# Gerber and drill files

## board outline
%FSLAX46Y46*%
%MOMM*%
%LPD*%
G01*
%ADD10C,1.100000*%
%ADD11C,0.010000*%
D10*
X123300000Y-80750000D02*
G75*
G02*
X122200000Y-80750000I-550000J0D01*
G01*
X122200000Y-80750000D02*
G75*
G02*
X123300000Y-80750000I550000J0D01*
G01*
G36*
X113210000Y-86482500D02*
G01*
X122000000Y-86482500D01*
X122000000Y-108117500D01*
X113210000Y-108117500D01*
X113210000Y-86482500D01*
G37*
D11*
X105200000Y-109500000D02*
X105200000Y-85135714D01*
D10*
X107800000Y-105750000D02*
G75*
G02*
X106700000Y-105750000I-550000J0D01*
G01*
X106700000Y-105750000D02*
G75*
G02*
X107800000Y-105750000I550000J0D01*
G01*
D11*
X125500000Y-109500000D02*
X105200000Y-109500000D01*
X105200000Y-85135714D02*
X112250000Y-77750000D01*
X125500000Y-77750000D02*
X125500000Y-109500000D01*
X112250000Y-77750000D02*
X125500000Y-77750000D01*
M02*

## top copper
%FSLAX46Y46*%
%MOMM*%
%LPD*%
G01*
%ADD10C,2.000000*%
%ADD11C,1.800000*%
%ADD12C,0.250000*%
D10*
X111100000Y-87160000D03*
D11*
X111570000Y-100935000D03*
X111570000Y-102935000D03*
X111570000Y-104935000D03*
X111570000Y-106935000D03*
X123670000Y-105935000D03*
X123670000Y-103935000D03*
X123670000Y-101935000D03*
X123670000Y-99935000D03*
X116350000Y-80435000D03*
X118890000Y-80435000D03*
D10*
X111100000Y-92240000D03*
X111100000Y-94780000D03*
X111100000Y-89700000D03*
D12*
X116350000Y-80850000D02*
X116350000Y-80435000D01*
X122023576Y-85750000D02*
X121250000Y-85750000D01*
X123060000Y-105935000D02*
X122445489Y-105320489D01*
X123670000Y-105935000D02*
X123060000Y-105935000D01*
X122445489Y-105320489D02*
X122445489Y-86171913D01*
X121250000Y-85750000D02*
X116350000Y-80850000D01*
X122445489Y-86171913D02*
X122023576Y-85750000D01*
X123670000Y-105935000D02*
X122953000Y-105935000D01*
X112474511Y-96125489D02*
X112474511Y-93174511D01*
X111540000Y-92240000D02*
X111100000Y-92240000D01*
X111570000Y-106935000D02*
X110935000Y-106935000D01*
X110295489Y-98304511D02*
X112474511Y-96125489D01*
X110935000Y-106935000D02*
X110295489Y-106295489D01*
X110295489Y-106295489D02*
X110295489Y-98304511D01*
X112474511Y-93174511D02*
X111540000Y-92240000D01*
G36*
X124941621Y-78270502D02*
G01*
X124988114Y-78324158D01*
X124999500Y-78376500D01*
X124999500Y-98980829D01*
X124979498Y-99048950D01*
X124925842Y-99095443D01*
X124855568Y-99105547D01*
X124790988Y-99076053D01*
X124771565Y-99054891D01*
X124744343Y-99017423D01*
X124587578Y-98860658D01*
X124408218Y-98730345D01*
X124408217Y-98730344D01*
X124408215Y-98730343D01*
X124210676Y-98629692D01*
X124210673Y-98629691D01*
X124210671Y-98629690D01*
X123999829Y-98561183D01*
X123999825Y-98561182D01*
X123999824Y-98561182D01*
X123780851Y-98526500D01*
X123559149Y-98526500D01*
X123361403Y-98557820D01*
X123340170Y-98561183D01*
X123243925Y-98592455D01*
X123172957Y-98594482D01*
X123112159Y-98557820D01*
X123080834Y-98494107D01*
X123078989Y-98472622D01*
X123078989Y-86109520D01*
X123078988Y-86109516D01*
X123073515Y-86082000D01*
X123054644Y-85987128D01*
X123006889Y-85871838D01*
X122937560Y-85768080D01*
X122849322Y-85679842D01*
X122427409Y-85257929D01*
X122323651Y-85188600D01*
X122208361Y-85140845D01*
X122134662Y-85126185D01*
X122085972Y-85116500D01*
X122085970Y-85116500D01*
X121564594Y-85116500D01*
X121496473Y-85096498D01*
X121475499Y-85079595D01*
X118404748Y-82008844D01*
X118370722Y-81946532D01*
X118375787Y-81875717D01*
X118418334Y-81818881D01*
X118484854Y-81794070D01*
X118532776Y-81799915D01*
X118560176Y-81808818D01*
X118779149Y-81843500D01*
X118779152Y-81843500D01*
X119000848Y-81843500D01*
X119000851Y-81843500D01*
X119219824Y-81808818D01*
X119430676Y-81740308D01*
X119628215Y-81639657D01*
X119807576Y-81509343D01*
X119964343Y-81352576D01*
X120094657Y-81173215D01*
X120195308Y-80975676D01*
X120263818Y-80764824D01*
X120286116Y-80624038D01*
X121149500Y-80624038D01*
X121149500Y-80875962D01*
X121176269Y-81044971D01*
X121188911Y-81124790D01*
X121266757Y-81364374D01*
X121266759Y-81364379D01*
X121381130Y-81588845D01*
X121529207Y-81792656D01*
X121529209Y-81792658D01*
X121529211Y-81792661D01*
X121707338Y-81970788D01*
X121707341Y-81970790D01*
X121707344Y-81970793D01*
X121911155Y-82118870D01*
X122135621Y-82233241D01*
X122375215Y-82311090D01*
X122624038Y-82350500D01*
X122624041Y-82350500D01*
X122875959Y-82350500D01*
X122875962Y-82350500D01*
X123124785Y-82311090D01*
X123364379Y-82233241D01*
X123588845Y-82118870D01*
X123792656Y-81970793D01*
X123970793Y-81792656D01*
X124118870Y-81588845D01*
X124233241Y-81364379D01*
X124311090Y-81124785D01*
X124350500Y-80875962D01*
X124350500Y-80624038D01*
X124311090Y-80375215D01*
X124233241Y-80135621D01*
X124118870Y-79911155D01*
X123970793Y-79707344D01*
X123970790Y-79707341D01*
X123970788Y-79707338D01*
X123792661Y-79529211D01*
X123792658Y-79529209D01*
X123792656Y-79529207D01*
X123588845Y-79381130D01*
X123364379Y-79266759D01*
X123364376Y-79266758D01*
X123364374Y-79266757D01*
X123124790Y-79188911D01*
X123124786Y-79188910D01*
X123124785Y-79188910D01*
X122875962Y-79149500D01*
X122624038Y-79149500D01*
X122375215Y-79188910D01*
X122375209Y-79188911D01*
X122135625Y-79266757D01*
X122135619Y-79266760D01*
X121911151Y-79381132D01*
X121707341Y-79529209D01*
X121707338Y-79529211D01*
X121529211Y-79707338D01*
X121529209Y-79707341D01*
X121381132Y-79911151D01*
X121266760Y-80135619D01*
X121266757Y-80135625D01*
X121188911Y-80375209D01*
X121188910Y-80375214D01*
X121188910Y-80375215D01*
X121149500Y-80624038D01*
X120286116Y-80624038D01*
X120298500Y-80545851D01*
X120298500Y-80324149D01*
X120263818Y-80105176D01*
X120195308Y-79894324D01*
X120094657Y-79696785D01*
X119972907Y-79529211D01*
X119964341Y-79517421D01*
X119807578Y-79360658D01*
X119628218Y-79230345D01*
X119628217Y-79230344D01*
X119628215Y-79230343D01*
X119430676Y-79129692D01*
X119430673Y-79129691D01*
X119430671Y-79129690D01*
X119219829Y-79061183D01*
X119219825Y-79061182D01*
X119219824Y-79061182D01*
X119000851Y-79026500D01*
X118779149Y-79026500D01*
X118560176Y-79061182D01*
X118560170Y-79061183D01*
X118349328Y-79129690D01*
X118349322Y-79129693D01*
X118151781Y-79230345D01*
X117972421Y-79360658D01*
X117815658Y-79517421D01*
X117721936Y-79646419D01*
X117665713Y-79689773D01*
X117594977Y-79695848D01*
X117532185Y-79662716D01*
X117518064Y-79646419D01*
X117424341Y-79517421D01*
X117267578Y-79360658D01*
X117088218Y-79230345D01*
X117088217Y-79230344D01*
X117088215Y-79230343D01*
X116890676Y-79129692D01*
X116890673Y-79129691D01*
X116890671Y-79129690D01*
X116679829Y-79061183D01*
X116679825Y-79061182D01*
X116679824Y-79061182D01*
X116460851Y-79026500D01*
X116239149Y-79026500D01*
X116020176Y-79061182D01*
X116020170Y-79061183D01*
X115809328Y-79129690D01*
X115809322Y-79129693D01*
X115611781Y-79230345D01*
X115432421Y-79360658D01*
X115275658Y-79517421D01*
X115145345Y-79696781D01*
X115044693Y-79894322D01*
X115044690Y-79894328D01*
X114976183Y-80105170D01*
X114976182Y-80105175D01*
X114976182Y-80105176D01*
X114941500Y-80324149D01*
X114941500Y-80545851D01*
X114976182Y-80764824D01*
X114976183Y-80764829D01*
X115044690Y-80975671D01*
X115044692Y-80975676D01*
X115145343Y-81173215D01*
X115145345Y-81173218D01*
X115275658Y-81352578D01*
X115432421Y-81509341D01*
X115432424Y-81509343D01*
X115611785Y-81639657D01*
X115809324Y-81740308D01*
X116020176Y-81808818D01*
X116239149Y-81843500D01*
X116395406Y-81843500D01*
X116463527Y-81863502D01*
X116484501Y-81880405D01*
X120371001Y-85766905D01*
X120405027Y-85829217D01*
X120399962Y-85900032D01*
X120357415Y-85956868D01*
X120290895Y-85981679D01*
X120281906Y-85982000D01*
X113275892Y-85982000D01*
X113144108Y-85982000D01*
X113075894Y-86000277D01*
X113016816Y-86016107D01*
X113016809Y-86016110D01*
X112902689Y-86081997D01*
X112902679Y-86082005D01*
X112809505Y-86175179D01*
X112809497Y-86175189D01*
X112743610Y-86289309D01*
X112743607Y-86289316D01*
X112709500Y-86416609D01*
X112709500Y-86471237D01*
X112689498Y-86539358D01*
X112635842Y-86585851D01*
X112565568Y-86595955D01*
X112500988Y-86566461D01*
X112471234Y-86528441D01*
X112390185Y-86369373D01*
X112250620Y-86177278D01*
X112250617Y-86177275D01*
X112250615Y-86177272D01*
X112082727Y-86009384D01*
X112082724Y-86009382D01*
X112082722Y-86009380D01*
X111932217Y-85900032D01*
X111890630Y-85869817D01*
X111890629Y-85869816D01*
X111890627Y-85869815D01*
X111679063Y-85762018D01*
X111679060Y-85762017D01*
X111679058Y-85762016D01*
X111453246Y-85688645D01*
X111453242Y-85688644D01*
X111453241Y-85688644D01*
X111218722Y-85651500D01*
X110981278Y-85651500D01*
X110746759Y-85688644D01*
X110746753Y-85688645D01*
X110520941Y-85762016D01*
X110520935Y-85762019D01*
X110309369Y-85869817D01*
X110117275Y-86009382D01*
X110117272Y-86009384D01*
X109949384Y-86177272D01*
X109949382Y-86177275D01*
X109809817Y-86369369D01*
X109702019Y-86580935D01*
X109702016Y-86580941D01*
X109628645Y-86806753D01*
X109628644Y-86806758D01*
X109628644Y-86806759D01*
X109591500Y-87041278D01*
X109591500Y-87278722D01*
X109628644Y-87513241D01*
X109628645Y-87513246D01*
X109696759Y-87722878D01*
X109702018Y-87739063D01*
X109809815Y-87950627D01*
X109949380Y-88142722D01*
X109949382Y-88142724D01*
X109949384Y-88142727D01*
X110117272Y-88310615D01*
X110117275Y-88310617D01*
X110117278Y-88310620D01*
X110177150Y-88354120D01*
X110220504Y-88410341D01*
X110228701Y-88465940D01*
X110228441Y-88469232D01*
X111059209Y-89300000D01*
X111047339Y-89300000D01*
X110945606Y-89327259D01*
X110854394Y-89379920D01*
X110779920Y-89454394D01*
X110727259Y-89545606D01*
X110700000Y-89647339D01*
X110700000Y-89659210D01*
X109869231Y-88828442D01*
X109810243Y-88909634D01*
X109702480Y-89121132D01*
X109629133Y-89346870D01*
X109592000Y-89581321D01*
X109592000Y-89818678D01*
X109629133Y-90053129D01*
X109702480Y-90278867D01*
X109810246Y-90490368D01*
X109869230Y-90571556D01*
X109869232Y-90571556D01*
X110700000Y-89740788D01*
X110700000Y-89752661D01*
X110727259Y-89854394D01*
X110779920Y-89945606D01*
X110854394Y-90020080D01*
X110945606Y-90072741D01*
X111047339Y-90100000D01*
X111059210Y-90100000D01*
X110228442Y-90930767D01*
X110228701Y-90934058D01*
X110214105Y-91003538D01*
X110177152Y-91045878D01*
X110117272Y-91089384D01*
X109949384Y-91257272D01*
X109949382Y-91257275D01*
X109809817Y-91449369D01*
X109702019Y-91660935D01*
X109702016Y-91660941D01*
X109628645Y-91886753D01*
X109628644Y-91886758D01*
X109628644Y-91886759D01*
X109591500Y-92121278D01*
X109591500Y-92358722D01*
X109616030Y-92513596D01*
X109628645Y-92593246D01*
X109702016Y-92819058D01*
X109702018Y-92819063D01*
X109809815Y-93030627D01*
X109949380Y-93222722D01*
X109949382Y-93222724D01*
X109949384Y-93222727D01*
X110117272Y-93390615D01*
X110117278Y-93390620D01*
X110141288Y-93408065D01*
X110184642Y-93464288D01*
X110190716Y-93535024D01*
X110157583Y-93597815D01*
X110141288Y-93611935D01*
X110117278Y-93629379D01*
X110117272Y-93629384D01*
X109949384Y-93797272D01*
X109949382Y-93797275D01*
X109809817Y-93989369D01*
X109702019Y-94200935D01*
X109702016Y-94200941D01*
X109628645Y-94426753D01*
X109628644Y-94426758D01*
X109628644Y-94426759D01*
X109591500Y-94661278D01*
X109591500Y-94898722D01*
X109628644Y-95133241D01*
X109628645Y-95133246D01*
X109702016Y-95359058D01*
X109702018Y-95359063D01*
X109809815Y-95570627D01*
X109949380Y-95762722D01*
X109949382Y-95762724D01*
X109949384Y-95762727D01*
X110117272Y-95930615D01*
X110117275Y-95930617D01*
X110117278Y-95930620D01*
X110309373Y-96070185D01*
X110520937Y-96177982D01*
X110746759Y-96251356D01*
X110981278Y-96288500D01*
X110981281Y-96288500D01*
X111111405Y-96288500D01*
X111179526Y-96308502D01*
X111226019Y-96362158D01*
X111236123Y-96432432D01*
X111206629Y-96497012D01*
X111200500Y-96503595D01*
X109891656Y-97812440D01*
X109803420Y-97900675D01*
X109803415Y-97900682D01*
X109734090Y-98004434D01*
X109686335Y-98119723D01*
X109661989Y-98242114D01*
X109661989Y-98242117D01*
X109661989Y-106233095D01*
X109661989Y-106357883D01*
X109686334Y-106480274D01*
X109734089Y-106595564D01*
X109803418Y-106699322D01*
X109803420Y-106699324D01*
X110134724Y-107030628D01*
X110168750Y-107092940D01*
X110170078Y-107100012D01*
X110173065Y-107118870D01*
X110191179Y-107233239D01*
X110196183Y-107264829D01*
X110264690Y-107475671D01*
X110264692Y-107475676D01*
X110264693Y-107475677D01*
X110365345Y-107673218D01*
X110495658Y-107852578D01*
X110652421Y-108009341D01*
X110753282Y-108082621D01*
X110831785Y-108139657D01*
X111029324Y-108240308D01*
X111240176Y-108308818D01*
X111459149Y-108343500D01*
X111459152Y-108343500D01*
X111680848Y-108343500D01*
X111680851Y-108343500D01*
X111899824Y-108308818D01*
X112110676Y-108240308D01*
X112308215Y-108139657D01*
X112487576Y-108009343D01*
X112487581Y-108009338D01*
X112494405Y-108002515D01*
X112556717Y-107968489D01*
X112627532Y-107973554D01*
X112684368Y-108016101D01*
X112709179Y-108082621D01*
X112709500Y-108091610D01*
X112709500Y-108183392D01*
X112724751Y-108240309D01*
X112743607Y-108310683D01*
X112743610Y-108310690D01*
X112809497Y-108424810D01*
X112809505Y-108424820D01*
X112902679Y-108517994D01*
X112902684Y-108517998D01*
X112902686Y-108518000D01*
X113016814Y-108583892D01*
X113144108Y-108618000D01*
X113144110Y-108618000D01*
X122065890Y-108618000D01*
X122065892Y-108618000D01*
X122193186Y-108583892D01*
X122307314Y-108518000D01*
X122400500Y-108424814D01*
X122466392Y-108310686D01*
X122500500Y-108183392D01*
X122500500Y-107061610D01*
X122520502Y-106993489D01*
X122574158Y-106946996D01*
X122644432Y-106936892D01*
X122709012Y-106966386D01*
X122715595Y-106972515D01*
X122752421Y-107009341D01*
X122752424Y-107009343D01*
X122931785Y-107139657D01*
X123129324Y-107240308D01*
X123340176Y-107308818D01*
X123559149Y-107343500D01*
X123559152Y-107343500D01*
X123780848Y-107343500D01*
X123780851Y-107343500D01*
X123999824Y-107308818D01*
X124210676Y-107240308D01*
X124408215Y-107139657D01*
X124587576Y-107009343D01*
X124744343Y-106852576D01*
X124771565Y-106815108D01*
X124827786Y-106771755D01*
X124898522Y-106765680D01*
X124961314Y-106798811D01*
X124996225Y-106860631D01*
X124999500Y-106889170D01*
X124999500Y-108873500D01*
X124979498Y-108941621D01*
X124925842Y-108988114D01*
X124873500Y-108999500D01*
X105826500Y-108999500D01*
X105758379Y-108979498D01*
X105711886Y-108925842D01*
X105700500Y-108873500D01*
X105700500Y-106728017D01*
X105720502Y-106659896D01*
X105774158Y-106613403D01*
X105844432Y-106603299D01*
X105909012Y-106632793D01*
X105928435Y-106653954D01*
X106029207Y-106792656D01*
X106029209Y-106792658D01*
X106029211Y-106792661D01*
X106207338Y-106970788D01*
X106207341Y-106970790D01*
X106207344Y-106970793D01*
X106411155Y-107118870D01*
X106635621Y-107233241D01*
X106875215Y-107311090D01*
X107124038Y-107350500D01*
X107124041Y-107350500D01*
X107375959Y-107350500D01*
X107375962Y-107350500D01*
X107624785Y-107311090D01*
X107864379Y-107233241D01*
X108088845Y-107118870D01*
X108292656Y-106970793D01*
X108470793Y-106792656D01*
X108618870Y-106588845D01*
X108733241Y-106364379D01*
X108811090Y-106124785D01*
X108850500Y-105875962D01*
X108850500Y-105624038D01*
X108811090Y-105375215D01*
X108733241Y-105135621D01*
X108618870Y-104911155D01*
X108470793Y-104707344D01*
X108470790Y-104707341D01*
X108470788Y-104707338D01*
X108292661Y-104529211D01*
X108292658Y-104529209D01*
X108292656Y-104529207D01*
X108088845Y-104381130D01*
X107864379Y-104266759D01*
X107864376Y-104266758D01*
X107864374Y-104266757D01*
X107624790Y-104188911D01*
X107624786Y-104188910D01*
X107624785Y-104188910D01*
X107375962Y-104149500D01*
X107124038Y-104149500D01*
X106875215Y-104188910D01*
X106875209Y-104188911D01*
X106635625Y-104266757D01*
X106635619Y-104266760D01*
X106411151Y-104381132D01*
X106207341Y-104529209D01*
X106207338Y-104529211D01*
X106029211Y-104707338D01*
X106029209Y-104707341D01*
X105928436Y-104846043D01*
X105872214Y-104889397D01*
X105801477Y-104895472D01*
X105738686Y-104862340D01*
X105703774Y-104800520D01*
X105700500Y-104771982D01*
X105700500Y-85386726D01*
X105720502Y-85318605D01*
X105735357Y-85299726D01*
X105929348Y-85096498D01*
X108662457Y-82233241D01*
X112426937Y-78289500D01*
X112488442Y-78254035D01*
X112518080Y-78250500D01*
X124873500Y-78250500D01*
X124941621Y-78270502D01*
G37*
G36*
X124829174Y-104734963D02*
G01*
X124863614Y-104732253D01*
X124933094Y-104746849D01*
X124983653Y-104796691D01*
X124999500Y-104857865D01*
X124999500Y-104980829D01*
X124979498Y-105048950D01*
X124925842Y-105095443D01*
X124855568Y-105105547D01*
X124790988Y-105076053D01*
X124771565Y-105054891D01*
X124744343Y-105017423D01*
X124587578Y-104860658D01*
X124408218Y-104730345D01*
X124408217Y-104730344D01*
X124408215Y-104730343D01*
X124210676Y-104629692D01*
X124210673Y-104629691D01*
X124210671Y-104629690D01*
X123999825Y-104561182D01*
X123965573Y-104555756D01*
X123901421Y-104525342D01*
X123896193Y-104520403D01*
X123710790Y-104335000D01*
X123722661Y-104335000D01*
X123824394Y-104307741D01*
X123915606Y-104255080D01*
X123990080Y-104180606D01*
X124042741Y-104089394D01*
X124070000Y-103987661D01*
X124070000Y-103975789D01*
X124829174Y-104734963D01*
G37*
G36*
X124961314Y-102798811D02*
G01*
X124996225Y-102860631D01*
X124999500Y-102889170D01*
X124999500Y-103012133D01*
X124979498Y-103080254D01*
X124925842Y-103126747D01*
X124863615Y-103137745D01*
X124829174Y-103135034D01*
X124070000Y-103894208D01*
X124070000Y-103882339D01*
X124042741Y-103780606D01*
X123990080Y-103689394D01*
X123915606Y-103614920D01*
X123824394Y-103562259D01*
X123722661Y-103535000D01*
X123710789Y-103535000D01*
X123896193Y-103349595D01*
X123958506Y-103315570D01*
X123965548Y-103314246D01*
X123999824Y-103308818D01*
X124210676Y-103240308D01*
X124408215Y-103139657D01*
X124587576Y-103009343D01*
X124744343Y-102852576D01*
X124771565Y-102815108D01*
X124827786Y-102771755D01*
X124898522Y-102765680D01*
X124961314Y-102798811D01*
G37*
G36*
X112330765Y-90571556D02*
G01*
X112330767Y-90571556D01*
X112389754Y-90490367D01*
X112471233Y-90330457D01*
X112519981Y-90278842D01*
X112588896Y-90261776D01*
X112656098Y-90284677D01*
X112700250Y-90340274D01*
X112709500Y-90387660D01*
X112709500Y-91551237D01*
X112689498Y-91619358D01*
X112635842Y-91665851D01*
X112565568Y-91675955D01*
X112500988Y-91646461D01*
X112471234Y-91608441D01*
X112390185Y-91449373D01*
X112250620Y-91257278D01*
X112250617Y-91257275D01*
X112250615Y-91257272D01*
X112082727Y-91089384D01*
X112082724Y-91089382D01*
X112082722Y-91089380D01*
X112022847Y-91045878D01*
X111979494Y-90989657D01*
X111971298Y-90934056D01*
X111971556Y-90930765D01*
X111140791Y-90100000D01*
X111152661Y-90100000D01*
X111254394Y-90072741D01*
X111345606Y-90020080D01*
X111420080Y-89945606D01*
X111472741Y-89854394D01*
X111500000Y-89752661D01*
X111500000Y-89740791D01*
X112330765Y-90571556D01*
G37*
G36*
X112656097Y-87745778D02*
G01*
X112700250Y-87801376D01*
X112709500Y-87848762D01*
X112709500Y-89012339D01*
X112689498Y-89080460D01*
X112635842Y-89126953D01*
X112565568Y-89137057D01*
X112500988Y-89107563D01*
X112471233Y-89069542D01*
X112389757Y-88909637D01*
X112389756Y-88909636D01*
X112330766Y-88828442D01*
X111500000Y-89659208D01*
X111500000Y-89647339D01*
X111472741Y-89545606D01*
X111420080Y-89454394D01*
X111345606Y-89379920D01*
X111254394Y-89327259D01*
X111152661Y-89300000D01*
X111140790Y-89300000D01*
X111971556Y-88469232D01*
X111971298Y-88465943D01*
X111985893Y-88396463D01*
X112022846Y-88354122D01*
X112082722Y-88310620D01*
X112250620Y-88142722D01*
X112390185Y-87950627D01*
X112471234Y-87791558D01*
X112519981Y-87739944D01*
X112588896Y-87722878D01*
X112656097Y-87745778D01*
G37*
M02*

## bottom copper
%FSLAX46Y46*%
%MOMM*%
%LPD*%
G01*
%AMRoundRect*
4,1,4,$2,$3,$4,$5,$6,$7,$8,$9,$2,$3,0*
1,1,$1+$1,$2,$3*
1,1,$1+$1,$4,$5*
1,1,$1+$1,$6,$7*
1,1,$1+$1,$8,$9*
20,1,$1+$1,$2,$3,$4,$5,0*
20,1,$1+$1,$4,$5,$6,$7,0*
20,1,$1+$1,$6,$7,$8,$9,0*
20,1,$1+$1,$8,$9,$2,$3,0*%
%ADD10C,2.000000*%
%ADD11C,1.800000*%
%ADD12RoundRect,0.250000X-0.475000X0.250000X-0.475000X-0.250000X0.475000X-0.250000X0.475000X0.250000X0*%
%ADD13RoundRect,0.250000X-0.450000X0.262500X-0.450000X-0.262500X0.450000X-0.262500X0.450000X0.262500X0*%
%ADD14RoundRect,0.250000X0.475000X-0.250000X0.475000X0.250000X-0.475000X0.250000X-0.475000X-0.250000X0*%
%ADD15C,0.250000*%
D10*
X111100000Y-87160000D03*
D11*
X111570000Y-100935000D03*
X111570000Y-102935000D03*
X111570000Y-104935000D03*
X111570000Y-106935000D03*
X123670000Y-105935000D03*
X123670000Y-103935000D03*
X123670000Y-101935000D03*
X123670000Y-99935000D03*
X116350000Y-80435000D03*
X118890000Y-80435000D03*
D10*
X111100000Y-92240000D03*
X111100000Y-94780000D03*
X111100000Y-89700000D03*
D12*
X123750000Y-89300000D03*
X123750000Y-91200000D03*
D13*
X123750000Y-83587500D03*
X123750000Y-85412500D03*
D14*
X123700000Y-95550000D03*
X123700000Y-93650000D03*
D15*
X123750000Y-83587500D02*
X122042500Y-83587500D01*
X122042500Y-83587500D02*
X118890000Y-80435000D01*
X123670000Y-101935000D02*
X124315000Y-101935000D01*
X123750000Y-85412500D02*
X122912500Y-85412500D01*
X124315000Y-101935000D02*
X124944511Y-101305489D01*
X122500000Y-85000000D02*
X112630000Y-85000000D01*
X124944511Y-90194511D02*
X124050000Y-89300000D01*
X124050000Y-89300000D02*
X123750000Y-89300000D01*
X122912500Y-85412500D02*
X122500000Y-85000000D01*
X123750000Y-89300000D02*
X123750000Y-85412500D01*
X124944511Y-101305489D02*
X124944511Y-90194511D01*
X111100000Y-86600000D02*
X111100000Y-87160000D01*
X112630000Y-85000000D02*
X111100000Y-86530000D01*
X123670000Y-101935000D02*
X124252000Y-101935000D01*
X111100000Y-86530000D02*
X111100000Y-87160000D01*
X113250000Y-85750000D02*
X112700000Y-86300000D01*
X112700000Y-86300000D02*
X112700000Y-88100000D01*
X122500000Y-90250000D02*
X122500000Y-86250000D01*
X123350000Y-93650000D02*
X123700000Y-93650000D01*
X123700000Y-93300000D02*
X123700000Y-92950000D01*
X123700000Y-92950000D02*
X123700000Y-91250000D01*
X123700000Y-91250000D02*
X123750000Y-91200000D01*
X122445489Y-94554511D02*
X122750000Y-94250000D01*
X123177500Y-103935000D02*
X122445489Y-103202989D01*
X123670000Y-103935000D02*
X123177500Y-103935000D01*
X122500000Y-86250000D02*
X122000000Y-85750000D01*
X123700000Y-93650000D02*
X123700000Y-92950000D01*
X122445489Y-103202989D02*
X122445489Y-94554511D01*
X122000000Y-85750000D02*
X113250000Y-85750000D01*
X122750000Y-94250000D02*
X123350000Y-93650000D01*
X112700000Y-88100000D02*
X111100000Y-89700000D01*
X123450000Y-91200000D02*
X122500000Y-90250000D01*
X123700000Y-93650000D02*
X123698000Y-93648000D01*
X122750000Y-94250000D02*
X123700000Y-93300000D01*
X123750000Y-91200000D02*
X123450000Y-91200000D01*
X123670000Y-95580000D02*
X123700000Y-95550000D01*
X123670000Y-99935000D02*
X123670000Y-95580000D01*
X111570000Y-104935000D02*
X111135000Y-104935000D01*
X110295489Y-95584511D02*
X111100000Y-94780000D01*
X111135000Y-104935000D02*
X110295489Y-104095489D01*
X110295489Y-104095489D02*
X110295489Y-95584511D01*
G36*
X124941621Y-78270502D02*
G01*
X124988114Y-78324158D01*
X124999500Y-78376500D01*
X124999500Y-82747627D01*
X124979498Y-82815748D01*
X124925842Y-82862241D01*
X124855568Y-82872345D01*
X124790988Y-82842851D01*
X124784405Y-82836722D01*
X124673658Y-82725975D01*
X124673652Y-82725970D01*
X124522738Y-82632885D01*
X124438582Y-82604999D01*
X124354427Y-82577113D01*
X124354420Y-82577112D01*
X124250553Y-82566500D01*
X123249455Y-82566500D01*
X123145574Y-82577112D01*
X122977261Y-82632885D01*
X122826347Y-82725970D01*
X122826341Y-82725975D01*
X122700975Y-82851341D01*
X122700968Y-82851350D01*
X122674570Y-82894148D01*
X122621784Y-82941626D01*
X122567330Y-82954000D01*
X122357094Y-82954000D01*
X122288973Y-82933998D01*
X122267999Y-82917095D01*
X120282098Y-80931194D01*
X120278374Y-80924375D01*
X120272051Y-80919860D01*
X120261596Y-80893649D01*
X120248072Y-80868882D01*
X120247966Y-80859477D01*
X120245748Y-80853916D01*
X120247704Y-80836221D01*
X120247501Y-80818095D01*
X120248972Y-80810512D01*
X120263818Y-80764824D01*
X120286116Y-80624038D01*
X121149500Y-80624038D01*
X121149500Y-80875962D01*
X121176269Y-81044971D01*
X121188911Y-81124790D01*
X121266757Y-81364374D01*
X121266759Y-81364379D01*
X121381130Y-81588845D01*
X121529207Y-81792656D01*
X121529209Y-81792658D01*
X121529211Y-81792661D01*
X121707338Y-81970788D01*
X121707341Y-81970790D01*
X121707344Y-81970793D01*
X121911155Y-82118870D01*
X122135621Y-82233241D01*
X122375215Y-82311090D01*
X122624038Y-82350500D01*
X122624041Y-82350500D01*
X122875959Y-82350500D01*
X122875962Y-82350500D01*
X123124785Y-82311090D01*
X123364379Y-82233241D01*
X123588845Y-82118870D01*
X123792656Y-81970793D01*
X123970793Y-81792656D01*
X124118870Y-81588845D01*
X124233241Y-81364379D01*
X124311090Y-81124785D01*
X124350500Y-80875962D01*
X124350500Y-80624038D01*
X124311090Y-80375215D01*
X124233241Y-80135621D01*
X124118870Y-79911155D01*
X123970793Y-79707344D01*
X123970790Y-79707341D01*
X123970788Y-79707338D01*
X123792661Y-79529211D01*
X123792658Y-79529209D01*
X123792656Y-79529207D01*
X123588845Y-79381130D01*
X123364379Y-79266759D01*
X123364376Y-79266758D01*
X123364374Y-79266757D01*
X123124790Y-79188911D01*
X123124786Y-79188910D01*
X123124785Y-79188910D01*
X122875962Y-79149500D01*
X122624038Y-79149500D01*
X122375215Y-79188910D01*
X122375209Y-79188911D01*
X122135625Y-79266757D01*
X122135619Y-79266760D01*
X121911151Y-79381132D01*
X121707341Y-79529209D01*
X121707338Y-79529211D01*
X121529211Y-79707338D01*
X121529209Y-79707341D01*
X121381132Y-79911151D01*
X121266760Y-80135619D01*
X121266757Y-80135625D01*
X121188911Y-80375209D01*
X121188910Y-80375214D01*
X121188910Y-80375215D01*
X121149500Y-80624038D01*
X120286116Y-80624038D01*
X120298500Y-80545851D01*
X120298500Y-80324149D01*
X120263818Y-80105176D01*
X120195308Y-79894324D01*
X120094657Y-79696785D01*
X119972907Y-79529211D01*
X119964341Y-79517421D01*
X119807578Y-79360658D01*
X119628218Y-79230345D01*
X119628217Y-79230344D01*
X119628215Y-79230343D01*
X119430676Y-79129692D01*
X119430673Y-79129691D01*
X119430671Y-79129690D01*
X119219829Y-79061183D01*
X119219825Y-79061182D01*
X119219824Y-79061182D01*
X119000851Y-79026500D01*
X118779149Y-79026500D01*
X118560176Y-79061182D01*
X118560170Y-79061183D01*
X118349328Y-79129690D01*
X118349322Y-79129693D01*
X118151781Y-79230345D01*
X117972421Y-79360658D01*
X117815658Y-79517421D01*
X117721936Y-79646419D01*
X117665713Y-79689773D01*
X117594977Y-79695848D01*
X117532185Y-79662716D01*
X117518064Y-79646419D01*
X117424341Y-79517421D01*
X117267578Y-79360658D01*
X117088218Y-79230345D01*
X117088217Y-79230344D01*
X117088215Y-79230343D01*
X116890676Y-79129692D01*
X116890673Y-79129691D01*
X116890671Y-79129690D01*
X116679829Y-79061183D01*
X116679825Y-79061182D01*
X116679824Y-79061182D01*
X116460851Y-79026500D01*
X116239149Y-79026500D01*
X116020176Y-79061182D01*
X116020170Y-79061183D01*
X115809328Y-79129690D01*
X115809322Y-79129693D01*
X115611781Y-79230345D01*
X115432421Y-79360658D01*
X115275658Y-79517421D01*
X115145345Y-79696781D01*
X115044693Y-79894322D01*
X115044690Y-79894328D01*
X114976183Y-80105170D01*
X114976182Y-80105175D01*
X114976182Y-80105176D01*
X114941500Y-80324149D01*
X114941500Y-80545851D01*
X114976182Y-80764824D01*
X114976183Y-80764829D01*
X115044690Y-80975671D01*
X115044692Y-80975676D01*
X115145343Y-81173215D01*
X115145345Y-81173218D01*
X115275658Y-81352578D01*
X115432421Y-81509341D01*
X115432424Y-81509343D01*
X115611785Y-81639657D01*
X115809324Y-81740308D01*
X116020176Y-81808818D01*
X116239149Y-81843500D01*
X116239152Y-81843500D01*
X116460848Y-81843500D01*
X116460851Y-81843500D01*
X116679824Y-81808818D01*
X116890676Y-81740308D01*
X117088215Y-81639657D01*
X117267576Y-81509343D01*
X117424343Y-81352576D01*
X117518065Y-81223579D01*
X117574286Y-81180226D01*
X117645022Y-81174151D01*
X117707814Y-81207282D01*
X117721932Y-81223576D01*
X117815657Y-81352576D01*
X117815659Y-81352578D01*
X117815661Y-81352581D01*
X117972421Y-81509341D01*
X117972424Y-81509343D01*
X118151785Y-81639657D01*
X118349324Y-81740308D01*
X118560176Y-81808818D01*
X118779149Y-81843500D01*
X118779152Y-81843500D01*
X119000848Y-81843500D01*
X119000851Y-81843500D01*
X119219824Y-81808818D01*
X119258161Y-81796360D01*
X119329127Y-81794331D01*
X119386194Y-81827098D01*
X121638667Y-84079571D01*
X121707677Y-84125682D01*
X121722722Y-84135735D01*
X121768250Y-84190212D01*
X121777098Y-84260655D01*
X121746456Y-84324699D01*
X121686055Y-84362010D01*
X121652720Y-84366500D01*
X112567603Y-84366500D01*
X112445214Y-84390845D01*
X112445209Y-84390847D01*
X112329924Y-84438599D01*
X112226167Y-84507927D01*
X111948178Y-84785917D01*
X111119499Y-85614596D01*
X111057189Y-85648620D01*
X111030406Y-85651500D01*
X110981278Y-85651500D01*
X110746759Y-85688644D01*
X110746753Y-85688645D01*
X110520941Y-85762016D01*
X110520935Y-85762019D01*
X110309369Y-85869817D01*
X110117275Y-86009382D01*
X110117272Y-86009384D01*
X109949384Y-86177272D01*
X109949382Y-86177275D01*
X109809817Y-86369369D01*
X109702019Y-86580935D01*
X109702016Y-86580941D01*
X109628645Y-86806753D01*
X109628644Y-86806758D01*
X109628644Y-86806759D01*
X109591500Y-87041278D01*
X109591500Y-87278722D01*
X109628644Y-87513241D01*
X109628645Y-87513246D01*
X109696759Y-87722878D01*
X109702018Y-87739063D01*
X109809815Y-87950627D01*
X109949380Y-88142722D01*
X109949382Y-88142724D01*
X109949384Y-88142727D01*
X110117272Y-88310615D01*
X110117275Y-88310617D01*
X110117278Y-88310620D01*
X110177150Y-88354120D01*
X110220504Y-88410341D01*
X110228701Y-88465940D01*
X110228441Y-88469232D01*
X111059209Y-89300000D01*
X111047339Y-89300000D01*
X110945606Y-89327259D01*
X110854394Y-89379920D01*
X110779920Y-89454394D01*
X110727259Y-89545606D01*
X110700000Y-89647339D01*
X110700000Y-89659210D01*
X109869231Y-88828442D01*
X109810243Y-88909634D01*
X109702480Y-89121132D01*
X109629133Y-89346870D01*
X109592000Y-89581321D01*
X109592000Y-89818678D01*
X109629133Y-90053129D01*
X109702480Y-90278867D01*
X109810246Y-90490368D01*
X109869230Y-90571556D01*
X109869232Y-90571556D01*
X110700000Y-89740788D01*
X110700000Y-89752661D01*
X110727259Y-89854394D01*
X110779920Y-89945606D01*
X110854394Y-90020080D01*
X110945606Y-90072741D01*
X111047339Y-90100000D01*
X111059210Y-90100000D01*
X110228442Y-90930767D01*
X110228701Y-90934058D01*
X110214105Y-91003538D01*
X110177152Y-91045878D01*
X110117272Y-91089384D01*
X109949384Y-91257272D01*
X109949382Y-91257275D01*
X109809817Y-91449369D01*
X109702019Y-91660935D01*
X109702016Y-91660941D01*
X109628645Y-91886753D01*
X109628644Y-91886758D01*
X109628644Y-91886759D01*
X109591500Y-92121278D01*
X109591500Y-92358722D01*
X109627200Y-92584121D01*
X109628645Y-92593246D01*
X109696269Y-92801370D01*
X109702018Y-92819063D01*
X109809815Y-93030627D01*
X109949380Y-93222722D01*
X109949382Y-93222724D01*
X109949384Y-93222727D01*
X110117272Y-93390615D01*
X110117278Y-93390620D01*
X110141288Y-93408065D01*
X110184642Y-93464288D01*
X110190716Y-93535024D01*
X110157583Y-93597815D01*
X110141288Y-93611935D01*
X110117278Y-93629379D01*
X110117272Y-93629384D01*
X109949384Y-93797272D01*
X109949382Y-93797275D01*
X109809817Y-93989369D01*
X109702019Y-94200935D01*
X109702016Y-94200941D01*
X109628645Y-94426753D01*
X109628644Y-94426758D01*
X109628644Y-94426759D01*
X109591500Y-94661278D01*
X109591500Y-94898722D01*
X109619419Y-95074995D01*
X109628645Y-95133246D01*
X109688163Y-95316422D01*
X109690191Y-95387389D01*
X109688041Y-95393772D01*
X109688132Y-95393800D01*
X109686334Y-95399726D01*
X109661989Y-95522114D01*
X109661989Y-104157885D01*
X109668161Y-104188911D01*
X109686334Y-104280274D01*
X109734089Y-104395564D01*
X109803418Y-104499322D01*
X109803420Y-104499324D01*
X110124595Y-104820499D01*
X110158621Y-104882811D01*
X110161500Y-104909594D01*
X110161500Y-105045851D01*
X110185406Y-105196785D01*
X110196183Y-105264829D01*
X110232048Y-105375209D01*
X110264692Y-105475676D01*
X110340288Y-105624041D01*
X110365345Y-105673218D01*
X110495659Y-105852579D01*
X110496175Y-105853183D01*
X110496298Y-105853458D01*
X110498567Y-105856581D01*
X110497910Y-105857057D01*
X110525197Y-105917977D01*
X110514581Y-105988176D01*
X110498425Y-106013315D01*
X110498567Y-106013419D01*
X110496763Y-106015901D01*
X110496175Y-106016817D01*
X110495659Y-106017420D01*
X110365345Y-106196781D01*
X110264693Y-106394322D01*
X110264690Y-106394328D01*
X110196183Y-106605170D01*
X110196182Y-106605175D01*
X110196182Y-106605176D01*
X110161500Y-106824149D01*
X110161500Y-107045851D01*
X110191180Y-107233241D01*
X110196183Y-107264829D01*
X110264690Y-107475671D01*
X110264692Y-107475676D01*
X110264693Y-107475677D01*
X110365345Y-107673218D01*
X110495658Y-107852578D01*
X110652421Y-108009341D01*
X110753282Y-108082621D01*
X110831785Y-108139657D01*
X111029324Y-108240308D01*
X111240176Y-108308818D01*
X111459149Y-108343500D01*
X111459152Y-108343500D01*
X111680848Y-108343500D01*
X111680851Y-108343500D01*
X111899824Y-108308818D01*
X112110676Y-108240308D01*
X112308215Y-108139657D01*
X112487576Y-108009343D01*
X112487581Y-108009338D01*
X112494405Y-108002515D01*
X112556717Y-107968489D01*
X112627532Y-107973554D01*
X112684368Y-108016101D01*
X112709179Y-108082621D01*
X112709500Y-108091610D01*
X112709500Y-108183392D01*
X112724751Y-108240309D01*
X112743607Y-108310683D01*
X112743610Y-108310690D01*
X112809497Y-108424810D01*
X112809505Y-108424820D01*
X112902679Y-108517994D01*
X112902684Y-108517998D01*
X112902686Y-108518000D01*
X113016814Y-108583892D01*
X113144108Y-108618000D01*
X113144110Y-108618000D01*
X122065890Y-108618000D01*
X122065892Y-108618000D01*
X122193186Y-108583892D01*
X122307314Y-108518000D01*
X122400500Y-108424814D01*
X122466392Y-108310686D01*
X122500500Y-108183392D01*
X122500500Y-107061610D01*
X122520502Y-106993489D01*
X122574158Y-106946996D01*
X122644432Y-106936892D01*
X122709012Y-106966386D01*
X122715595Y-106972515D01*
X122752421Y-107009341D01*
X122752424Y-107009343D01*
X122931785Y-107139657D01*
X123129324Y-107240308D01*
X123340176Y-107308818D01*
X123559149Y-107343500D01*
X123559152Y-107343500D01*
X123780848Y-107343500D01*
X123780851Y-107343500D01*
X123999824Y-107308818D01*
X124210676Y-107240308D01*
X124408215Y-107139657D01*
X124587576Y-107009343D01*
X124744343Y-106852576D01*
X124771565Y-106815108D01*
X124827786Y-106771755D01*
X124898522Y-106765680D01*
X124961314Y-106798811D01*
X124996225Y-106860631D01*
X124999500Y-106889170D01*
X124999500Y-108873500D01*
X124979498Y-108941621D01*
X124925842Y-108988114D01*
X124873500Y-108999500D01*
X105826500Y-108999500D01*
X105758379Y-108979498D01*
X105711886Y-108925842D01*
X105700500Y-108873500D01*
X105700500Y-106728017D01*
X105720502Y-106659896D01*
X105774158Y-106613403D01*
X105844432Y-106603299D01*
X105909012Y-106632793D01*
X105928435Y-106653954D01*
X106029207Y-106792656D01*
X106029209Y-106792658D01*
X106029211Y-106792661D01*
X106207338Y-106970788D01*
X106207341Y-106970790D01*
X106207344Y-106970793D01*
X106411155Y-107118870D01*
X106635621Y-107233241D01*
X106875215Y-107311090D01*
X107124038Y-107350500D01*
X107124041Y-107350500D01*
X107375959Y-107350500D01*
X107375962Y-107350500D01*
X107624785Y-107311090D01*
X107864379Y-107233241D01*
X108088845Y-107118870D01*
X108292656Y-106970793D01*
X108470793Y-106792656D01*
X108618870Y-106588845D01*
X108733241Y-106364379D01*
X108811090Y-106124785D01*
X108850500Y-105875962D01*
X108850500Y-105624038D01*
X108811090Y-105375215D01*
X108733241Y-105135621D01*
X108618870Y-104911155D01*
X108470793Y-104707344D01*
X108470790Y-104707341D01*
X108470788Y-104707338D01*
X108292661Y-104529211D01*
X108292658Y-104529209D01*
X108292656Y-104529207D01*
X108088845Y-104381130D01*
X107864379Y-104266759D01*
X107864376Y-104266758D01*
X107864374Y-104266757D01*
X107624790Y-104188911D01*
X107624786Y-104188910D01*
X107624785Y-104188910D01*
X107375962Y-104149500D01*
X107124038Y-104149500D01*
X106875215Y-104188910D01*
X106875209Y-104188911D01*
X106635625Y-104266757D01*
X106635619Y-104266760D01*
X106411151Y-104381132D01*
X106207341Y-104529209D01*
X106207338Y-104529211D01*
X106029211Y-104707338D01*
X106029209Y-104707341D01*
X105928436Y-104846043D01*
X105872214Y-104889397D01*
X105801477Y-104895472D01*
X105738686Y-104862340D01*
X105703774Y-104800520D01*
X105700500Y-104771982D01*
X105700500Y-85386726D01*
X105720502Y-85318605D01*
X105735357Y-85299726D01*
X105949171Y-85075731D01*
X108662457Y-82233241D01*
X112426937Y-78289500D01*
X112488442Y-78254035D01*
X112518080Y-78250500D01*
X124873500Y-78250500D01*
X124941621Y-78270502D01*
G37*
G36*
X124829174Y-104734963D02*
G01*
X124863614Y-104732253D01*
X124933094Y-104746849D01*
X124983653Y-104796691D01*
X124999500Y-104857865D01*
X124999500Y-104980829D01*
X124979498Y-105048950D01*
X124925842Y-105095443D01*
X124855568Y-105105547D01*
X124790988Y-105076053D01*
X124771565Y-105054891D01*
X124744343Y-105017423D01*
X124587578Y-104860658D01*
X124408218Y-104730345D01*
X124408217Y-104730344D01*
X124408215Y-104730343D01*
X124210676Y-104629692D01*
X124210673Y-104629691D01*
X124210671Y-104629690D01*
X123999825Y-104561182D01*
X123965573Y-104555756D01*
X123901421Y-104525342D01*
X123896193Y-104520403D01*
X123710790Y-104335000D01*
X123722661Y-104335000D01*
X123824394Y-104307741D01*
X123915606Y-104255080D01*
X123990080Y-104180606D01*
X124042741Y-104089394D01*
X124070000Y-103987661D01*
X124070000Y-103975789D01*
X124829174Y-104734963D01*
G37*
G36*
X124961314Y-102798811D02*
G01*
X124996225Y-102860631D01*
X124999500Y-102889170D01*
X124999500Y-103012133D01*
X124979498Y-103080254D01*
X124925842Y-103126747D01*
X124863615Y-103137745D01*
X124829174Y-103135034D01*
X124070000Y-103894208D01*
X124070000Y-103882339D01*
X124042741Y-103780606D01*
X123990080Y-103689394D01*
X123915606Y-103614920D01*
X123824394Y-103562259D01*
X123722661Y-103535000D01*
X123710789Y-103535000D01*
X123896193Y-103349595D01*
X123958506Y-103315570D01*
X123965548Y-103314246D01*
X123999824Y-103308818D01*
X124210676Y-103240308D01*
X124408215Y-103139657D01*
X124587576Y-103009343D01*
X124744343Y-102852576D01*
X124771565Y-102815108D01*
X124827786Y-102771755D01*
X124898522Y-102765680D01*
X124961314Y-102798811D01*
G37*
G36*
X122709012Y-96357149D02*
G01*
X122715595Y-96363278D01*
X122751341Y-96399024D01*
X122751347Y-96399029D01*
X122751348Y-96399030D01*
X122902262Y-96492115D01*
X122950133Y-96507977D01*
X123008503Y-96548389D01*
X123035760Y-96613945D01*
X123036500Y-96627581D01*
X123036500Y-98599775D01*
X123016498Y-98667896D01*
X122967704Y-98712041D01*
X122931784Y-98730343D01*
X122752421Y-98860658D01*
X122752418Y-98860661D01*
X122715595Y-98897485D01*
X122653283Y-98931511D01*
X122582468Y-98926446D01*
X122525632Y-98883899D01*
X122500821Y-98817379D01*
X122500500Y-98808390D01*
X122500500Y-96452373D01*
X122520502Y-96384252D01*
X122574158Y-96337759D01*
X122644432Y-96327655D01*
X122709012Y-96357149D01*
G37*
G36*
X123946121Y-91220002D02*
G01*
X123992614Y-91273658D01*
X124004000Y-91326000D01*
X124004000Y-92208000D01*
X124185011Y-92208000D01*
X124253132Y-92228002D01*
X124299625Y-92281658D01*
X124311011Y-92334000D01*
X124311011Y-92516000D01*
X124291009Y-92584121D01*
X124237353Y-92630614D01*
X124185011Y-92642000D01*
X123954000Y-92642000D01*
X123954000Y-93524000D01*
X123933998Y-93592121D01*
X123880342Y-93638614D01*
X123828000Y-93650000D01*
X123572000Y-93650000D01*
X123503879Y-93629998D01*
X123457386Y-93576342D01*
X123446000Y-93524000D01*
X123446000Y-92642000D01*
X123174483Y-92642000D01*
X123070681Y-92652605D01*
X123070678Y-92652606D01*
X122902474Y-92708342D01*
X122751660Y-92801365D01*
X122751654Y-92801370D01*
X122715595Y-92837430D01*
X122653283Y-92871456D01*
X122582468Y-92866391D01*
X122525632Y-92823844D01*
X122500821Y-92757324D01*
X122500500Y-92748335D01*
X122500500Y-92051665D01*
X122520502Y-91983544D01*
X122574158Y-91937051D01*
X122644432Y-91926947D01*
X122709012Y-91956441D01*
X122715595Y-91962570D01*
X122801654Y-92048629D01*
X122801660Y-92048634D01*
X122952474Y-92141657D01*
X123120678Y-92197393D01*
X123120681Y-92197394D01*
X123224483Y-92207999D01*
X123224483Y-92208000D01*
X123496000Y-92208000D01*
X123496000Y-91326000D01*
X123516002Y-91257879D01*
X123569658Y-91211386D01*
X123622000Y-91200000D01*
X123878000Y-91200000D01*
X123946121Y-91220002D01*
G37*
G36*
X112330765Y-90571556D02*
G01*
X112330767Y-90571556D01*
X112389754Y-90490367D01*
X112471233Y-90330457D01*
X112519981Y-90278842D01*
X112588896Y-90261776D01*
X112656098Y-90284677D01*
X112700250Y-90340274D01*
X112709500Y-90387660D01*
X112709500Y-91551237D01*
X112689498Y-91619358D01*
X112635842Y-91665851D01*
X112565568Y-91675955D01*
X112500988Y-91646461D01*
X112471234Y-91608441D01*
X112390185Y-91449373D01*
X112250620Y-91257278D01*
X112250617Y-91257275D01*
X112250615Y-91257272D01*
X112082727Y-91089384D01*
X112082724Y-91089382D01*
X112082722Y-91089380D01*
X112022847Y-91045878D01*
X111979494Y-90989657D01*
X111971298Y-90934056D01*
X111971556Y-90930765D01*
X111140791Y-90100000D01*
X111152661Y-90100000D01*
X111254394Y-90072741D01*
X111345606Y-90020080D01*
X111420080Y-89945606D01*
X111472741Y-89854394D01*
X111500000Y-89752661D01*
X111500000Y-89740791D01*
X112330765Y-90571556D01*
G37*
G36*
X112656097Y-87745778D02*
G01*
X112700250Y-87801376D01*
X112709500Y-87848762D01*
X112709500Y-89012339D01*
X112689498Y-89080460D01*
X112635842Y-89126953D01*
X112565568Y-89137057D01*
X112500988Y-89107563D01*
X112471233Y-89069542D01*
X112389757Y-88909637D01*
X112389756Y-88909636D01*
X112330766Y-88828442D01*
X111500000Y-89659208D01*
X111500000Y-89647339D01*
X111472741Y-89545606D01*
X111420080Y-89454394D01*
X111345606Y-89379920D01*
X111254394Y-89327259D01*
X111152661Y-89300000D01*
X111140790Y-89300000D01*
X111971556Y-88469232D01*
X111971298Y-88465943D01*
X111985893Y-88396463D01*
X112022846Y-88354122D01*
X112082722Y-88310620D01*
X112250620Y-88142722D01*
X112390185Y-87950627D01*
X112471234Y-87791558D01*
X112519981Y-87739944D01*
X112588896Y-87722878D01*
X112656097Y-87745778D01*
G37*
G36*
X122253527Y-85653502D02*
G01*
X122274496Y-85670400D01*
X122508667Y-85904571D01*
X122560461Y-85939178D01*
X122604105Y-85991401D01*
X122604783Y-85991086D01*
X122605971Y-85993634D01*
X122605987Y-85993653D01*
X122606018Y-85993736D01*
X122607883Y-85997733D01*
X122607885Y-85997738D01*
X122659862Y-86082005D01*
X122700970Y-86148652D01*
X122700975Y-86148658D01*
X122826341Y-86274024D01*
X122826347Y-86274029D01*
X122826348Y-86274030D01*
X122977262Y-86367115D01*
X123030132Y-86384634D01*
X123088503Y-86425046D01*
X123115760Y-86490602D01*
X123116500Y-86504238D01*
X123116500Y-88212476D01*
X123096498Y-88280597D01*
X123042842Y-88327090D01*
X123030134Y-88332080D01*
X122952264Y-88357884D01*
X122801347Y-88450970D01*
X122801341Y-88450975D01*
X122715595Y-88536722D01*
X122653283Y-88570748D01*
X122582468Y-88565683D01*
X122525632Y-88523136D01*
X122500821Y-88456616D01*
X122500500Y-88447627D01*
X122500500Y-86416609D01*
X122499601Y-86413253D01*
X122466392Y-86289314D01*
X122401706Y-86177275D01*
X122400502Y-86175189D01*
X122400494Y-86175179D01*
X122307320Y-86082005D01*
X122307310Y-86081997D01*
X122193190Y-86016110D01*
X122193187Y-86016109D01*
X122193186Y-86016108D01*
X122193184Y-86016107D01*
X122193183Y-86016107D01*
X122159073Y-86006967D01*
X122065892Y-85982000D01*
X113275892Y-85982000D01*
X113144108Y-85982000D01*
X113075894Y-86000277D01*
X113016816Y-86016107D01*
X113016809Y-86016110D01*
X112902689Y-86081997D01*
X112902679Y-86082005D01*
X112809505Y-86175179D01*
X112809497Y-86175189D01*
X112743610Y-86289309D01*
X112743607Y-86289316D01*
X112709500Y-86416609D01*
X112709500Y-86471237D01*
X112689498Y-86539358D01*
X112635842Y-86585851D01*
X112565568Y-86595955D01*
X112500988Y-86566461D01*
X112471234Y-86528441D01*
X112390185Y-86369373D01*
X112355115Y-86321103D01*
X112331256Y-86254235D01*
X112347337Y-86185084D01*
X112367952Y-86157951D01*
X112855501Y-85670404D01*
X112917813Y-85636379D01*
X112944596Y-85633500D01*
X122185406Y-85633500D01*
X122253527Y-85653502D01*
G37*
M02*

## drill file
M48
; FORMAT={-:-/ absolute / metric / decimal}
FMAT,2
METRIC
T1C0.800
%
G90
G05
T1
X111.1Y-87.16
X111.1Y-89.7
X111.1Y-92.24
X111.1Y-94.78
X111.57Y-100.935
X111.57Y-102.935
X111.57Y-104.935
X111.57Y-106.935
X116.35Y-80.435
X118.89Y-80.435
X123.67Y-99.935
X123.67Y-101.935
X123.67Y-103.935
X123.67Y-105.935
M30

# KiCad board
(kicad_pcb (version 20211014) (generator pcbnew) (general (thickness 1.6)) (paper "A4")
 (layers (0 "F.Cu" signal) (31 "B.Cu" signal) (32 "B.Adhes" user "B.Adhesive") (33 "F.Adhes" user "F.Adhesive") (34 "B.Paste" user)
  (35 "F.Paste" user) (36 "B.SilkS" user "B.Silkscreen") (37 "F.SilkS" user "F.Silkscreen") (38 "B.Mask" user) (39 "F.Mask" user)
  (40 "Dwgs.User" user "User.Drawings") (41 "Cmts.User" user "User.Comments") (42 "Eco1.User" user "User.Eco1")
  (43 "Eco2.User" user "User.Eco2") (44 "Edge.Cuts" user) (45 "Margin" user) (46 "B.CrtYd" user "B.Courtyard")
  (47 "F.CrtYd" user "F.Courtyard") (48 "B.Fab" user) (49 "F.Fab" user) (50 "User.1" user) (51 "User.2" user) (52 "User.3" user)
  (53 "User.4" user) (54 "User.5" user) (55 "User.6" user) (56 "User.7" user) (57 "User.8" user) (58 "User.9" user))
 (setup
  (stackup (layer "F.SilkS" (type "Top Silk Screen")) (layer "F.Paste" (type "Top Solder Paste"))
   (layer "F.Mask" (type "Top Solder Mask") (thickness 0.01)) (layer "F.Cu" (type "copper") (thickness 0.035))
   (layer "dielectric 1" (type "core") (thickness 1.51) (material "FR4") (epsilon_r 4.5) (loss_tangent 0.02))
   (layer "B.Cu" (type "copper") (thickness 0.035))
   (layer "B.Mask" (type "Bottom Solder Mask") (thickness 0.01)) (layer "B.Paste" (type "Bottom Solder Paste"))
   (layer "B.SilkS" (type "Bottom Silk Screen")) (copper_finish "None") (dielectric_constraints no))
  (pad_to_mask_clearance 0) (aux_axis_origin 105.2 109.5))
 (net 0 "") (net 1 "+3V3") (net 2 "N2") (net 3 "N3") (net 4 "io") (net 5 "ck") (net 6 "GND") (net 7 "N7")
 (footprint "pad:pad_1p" (layer "F.Cu") (at 111.1 87.16)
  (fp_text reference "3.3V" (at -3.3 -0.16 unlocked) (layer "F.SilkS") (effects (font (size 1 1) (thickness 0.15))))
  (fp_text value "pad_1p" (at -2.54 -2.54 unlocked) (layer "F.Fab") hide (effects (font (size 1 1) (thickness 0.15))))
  (pad "1" thru_hole circle (at 0 0) (size 2 2) (drill 0.8) (layers *.Cu *.Mask) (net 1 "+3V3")))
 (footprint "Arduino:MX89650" (layer "F.Cu") (at 117.62 102.935)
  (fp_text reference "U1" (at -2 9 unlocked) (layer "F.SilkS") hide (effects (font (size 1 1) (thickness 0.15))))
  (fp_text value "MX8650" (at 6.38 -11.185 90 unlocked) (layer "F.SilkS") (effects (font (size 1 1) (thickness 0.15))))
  (pad "1" thru_hole circle (at -6.05 -2) (size 1.8 1.8) (drill 0.8) (layers *.Cu *.Mask) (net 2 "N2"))
  (pad "2" thru_hole circle (at -6.05 0) (size 1.8 1.8) (drill 0.8) (layers *.Cu *.Mask) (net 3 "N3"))
  (pad "3" thru_hole circle (at -6.05 2) (size 1.8 1.8) (drill 0.8) (layers *.Cu *.Mask) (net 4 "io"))
  (pad "4" thru_hole circle (at -6.05 4) (size 1.8 1.8) (drill 0.8) (layers *.Cu *.Mask) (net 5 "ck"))
  (pad "5" thru_hole circle (at 6.05 3) (size 1.8 1.8) (drill 0.8) (layers *.Cu *.Mask))
  (pad "6" thru_hole circle (at 6.05 1) (size 1.8 1.8) (drill 0.8) (layers *.Cu *.Mask) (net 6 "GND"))
  (pad "7" thru_hole circle (at 6.05 -1) (size 1.8 1.8) (drill 0.8) (layers *.Cu *.Mask) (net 1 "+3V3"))
  (pad "8" thru_hole circle (at 6.05 -3) (size 1.8 1.8) (drill 0.8) (layers *.Cu *.Mask) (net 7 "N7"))
  (pad "9" thru_hole circle (at -1.27 -22.5) (size 1.8 1.8) (drill 0.8) (layers *.Cu *.Mask))
  (pad "10" thru_hole circle (at 1.27 -22.5) (size 1.8 1.8) (drill 0.8) (layers *.Cu *.Mask)))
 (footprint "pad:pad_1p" (layer "F.Cu") (at 111.1 92.24)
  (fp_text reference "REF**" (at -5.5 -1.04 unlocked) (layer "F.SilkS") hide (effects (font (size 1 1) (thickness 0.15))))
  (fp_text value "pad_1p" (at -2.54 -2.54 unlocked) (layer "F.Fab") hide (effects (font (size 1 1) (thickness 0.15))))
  (pad "1" thru_hole circle (at 0 0) (size 2 2) (drill 0.8) (layers *.Cu *.Mask) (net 5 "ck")))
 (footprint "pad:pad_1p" (layer "F.Cu") (at 111.1 94.78)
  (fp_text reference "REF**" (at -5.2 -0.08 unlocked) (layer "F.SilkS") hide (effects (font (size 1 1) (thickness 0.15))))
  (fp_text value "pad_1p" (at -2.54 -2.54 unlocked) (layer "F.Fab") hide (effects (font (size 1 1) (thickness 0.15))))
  (pad "1" thru_hole circle (at 0 0) (size 2 2) (drill 0.8) (layers *.Cu *.Mask) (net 4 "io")))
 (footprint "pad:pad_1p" (layer "F.Cu") (at 111.1 89.7)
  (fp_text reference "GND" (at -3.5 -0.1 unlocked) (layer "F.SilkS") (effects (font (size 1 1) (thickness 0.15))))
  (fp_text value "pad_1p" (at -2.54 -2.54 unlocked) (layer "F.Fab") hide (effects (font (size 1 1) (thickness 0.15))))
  (pad "1" thru_hole circle (at 0 0) (size 2 2) (drill 0.8) (layers *.Cu *.Mask) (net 6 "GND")))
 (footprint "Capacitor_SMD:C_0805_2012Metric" (layer "B.Cu") (at 123.75 90.25 -90)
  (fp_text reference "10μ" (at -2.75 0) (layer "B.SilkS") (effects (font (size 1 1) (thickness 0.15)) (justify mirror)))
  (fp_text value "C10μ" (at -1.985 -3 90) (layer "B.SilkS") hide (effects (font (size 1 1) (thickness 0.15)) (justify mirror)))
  (pad "1" smd roundrect (at -0.95 0 270) (size 1 1.45) (layers "B.Cu" "B.Paste" "B.Mask") (roundrect_rratio 0.25) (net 1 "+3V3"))
  (pad "2" smd roundrect (at 0.95 0 270) (size 1 1.45) (layers "B.Cu" "B.Paste" "B.Mask") (roundrect_rratio 0.25) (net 6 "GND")))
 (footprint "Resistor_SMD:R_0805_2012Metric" (layer "B.Cu") (at 123.75 84.5 -90)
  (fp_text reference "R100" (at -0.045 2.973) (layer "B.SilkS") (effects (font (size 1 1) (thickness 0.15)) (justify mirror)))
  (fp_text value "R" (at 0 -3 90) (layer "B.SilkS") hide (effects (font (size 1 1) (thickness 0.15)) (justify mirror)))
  (pad "1" smd roundrect (at -0.9125 0 270) (size 1.025 1.4) (layers "B.Cu" "B.Paste" "B.Mask") (roundrect_rratio 0.243902439))
  (pad "2" smd roundrect (at 0.9125 0 270) (size 1.025 1.4) (layers "B.Cu" "B.Paste" "B.Mask") (roundrect_rratio 0.243902439) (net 1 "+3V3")))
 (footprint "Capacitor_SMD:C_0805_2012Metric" (layer "B.Cu") (at 123.7 94.6 90)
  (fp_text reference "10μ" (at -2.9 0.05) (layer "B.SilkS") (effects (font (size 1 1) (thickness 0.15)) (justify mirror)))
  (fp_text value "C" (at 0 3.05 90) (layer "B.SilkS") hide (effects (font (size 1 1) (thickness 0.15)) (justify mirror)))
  (pad "1" smd roundrect (at -0.95 0 90) (size 1 1.45) (layers "B.Cu" "B.Paste" "B.Mask") (roundrect_rratio 0.25) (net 7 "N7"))
  (pad "2" smd roundrect (at 0.95 0 90) (size 1 1.45) (layers "B.Cu" "B.Paste" "B.Mask") (roundrect_rratio 0.25) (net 6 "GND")))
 (gr_circle (center 122.75 80.75) (end 123.85 80.75) (layer "Edge.Cuts") (width 0) (fill solid))
 (gr_rect (start 113.21 108.1175) (end 122 86.4825) (layer "Edge.Cuts") (width 0) (fill solid))
 (gr_line (start 105.2 109.5) (end 105.2 85.135714) (layer "Edge.Cuts") (width 0.01))
 (gr_circle (center 107.25 105.75) (end 108.35 105.75) (layer "Edge.Cuts") (width 0) (fill solid))
 (gr_line (start 125.5 109.5) (end 105.2 109.5) (layer "Edge.Cuts") (width 0.01))
 (gr_line (start 105.2 85.135714) (end 112.25 77.75) (layer "Edge.Cuts") (width 0.01))
 (gr_line (start 125.5 77.75) (end 125.5 109.5) (layer "Edge.Cuts") (width 0.01))
 (gr_line (start 112.25 77.75) (end 125.5 77.75) (layer "Edge.Cuts") (width 0.01))
 (segment (start 116.35 80.85) (end 116.35 80.435) (width 0.25) (layer "F.Cu") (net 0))
 (segment (start 122.023576 85.75) (end 121.25 85.75) (width 0.25) (layer "F.Cu") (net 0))
 (segment (start 123.06 105.935) (end 122.445489 105.320489) (width 0.25) (layer "F.Cu") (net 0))
 (segment (start 123.67 105.935) (end 123.06 105.935) (width 0.25) (layer "F.Cu") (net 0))
 (segment (start 122.445489 105.320489) (end 122.445489 86.171913) (width 0.25) (layer "F.Cu") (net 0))
 (segment (start 121.25 85.75) (end 116.35 80.85) (width 0.25) (layer "F.Cu") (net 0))
 (segment (start 122.445489 86.171913) (end 122.023576 85.75) (width 0.25) (layer "F.Cu") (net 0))
 (segment (start 123.67 105.935) (end 122.953 105.935) (width 0.25) (layer "F.Cu") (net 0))
 (segment (start 123.75 83.5875) (end 122.0425 83.5875) (width 0.25) (layer "B.Cu") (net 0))
 (segment (start 122.0425 83.5875) (end 118.89 80.435) (width 0.25) (layer "B.Cu") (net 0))
 (segment (start 123.67 101.935) (end 124.315 101.935) (width 0.25) (layer "B.Cu") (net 1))
 (segment (start 123.75 85.4125) (end 122.9125 85.4125) (width 0.25) (layer "B.Cu") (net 1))
 (segment (start 124.315 101.935) (end 124.944511 101.305489) (width 0.25) (layer "B.Cu") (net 1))
 (segment (start 122.5 85) (end 112.63 85) (width 0.25) (layer "B.Cu") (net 1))
 (segment (start 124.944511 90.194511) (end 124.05 89.3) (width 0.25) (layer "B.Cu") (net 1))
 (segment (start 124.05 89.3) (end 123.75 89.3) (width 0.25) (layer "B.Cu") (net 1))
 (segment (start 122.9125 85.4125) (end 122.5 85) (width 0.25) (layer "B.Cu") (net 1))
 (segment (start 123.75 89.3) (end 123.75 85.4125) (width 0.25) (layer "B.Cu") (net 1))
 (segment (start 124.944511 101.305489) (end 124.944511 90.194511) (width 0.25) (layer "B.Cu") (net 1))
 (segment (start 111.1 86.6) (end 111.1 87.16) (width 0.25) (layer "B.Cu") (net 1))
 (segment (start 112.63 85) (end 111.1 86.53) (width 0.25) (layer "B.Cu") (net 1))
 (segment (start 123.67 101.935) (end 124.252 101.935) (width 0.25) (layer "B.Cu") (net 1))
 (segment (start 111.1 86.53) (end 111.1 87.16) (width 0.25) (layer "B.Cu") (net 1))
 (segment (start 113.25 85.75) (end 112.7 86.3) (width 0.25) (layer "B.Cu") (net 6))
 (segment (start 112.7 86.3) (end 112.7 88.1) (width 0.25) (layer "B.Cu") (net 6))
 (segment (start 122.5 90.25) (end 122.5 86.25) (width 0.25) (layer "B.Cu") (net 6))
 (segment (start 123.35 93.65) (end 123.7 93.65) (width 0.25) (layer "B.Cu") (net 6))
 (segment (start 123.7 93.3) (end 123.7 92.95) (width 0.25) (layer "B.Cu") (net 6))
 (segment (start 123.7 92.95) (end 123.7 91.25) (width 0.25) (layer "B.Cu") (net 6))
 (segment (start 123.7 91.25) (end 123.75 91.2) (width 0.25) (layer "B.Cu") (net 6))
 (segment (start 122.445489 94.554511) (end 122.75 94.25) (width 0.25) (layer "B.Cu") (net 6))
 (segment (start 123.1775 103.935) (end 122.445489 103.202989) (width 0.25) (layer "B.Cu") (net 6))
 (segment (start 123.67 103.935) (end 123.1775 103.935) (width 0.25) (layer "B.Cu") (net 6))
 (segment (start 122.5 86.25) (end 122 85.75) (width 0.25) (layer "B.Cu") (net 6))
 (segment (start 123.7 93.65) (end 123.7 92.95) (width 0.25) (layer "B.Cu") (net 6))
 (segment (start 122.445489 103.202989) (end 122.445489 94.554511) (width 0.25) (layer "B.Cu") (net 6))
 (segment (start 122 85.75) (end 113.25 85.75) (width 0.25) (layer "B.Cu") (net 6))
 (segment (start 122.75 94.25) (end 123.35 93.65) (width 0.25) (layer "B.Cu") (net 6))
 (segment (start 112.7 88.1) (end 111.1 89.7) (width 0.25) (layer "B.Cu") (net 6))
 (segment (start 123.45 91.2) (end 122.5 90.25) (width 0.25) (layer "B.Cu") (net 6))
 (segment (start 123.7 93.65) (end 123.698 93.648) (width 0.25) (layer "B.Cu") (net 6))
 (segment (start 122.75 94.25) (end 123.7 93.3) (width 0.25) (layer "B.Cu") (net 6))
 (segment (start 123.75 91.2) (end 123.45 91.2) (width 0.25) (layer "B.Cu") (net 6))
 (segment (start 123.67 95.58) (end 123.7 95.55) (width 0.25) (layer "B.Cu") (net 7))
 (segment (start 123.67 99.935) (end 123.67 95.58) (width 0.25) (layer "B.Cu") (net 7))
 (segment (start 112.474511 96.125489) (end 112.474511 93.174511) (width 0.25) (layer "F.Cu") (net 5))
 (segment (start 111.54 92.24) (end 111.1 92.24) (width 0.25) (layer "F.Cu") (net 5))
 (segment (start 111.57 106.935) (end 110.935 106.935) (width 0.25) (layer "F.Cu") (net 5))
 (segment (start 110.295489 98.304511) (end 112.474511 96.125489) (width 0.25) (layer "F.Cu") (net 5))
 (segment (start 110.935 106.935) (end 110.295489 106.295489) (width 0.25) (layer "F.Cu") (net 5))
 (segment (start 110.295489 106.295489) (end 110.295489 98.304511) (width 0.25) (layer "F.Cu") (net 5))
 (segment (start 112.474511 93.174511) (end 111.54 92.24) (width 0.25) (layer "F.Cu") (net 5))
 (segment (start 111.57 104.935) (end 111.135 104.935) (width 0.25) (layer "B.Cu") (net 4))
 (segment (start 110.295489 95.584511) (end 111.1 94.78) (width 0.25) (layer "B.Cu") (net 4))
 (segment (start 111.135 104.935) (end 110.295489 104.095489) (width 0.25) (layer "B.Cu") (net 4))
 (segment (start 110.295489 104.095489) (end 110.295489 95.584511) (width 0.25) (layer "B.Cu") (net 4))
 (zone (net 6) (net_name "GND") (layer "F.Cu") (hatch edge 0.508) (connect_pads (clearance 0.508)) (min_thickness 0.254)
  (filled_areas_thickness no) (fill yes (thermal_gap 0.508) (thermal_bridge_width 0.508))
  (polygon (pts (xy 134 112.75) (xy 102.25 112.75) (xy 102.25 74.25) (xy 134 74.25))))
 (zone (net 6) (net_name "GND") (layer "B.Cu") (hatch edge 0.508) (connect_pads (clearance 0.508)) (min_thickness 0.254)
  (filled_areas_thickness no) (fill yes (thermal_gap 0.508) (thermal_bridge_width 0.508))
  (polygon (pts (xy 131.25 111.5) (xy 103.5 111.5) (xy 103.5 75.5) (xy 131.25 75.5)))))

